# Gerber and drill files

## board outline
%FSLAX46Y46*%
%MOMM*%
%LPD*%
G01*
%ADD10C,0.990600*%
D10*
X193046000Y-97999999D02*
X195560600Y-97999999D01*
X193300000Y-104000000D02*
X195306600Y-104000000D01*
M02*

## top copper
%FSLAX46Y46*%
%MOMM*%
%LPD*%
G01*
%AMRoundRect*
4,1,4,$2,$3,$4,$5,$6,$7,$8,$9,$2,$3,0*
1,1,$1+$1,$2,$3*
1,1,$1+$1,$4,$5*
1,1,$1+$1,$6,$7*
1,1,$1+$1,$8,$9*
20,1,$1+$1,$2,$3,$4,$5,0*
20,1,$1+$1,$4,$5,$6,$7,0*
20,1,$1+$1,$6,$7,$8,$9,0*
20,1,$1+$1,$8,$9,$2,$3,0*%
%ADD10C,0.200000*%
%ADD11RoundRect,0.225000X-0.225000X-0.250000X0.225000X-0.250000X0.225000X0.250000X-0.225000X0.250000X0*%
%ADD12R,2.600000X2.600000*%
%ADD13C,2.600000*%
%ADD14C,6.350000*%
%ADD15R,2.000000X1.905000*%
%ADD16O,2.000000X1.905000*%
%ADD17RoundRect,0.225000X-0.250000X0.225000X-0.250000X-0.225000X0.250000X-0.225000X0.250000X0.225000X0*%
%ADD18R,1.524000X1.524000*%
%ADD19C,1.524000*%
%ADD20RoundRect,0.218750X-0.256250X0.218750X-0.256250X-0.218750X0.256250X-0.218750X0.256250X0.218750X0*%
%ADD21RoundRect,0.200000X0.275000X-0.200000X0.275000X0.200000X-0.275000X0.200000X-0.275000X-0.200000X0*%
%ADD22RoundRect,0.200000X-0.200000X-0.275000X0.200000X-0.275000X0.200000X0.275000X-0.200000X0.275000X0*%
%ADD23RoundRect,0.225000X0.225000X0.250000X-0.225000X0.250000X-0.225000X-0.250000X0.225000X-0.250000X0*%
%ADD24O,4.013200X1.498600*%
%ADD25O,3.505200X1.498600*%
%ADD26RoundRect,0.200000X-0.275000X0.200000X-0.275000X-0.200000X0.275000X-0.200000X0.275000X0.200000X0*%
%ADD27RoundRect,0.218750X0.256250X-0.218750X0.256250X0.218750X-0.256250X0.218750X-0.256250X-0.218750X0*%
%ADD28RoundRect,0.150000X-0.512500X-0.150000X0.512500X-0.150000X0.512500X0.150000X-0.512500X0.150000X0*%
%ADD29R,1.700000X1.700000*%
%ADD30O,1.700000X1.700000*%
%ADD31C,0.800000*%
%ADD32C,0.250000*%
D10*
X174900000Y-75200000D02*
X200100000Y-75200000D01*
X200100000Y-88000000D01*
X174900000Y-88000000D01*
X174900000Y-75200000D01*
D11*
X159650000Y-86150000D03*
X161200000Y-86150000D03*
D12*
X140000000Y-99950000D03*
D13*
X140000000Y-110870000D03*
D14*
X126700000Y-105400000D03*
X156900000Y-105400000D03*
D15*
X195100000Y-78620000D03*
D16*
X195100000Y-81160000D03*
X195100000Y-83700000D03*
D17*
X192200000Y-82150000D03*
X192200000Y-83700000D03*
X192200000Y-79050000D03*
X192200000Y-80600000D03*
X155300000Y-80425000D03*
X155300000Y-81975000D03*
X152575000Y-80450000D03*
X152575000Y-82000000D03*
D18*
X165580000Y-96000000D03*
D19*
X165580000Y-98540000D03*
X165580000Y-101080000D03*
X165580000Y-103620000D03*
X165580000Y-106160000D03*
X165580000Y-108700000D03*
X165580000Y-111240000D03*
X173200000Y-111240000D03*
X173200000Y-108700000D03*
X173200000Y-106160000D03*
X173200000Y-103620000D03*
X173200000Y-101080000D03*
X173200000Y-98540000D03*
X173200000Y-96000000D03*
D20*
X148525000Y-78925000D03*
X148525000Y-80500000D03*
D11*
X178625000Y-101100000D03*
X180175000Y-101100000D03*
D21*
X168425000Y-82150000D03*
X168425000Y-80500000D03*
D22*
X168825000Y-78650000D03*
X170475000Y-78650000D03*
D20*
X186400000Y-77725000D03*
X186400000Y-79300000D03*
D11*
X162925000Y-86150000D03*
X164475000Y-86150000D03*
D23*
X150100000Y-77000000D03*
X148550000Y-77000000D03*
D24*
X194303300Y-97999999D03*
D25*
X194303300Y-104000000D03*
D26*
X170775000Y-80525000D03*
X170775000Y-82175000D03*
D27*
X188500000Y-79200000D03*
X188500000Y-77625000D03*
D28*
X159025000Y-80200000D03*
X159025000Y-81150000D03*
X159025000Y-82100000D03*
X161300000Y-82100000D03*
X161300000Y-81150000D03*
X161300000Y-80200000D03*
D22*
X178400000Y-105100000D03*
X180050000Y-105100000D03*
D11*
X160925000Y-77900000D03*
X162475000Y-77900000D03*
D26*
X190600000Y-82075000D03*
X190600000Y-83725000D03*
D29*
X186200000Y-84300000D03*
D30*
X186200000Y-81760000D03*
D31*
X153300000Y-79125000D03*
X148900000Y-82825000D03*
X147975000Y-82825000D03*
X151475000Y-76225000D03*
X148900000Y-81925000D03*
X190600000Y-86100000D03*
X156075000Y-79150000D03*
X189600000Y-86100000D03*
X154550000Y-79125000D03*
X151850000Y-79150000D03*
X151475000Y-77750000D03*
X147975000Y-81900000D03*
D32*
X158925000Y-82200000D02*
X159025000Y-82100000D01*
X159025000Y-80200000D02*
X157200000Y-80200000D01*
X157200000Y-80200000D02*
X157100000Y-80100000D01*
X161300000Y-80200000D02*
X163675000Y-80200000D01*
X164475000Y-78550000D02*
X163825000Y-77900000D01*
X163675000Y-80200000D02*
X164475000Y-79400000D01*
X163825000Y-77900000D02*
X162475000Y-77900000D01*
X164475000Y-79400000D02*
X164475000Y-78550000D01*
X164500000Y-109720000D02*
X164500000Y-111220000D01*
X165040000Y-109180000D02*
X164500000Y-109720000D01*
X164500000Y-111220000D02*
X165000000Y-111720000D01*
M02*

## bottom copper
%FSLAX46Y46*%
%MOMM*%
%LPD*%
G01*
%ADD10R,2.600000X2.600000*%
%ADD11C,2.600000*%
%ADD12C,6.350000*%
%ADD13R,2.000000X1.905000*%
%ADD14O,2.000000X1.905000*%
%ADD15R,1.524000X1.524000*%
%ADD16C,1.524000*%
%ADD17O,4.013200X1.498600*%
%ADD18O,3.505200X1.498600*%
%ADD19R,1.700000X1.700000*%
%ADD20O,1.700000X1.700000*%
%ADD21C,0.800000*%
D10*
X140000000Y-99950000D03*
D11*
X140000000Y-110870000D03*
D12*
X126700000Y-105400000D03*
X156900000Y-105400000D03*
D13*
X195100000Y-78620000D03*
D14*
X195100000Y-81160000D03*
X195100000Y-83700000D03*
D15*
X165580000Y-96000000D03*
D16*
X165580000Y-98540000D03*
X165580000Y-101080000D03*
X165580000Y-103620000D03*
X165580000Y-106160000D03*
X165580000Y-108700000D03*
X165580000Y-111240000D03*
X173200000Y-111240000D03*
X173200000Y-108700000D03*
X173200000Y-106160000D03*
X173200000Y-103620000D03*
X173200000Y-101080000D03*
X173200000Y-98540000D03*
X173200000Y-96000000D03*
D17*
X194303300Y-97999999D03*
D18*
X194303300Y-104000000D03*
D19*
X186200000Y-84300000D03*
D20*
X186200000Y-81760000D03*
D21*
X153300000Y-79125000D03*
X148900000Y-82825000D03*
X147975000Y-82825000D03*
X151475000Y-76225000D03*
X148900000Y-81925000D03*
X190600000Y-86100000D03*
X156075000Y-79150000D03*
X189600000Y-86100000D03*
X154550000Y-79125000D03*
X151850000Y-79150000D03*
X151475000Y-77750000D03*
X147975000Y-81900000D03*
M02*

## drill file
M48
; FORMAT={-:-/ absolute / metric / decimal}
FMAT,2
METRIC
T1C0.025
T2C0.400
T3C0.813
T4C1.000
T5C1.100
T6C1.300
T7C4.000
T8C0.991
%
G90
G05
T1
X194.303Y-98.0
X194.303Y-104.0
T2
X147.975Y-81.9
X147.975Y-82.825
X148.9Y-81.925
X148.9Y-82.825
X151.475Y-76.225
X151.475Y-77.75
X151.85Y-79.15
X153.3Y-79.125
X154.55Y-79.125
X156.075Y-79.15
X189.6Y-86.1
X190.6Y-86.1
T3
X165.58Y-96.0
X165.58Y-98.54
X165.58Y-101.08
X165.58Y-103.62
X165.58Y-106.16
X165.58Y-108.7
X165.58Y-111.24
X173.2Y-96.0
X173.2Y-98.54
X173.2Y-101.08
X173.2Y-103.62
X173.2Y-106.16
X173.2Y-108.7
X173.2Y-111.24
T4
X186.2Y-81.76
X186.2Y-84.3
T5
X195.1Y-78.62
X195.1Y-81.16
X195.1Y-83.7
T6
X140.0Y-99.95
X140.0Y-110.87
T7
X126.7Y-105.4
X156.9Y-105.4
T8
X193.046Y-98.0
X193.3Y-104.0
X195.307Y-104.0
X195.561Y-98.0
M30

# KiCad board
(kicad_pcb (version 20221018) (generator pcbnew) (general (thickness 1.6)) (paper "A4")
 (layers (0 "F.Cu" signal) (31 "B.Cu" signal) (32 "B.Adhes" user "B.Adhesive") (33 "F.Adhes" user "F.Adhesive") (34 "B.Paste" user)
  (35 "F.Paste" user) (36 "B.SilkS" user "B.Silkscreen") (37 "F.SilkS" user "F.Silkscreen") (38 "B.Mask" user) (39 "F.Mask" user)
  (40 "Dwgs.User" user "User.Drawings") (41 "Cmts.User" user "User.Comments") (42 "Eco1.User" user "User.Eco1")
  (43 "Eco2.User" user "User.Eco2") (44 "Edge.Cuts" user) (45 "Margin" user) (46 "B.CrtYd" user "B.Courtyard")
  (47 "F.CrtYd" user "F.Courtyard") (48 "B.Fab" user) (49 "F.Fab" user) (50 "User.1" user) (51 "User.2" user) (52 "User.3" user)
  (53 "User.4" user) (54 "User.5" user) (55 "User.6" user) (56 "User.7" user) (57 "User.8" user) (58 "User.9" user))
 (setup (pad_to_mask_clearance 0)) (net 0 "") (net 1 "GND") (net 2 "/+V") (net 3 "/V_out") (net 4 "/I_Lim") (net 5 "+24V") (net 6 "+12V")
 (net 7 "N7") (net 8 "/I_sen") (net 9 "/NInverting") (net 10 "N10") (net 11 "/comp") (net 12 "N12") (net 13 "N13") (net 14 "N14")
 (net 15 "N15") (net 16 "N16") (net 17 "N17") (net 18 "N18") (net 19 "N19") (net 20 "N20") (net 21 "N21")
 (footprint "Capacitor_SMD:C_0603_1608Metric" (layer "F.Cu") (at 160.425 86.15)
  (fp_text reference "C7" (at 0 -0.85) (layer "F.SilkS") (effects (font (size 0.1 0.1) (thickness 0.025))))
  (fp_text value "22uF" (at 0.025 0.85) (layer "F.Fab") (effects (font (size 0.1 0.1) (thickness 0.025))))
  (pad "1" smd roundrect (at -0.775 0) (size 0.9 0.95) (layers "F.Cu" "F.Paste" "F.Mask") (roundrect_rratio 0.25) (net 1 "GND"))
  (pad "2" smd roundrect (at 0.775 0) (size 0.9 0.95) (layers "F.Cu" "F.Paste" "F.Mask") (roundrect_rratio 0.25) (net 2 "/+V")))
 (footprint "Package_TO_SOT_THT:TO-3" (layer "F.Cu") (at 140 99.95)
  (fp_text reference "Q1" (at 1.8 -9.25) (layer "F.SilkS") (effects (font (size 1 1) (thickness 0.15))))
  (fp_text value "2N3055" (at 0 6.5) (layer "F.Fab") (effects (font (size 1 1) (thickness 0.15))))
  (pad "1" thru_hole rect (at 0 0) (size 2.6 2.6) (drill 1.3) (layers "*.Cu" "*.Mask") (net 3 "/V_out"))
  (pad "2" thru_hole circle (at 0 10.92) (size 2.6 2.6) (drill 1.3) (layers "*.Cu" "*.Mask") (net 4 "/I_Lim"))
  (pad "3" thru_hole circle (at -13.3 5.45) (size 6.35 6.35) (drill 4) (layers "*.Cu" "*.Mask") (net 2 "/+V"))
  (pad "3" thru_hole circle (at 16.9 5.45) (size 6.35 6.35) (drill 4) (layers "*.Cu" "*.Mask") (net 2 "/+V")))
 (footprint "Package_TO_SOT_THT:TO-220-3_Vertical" (layer "F.Cu") (at 195.1 78.62 -90)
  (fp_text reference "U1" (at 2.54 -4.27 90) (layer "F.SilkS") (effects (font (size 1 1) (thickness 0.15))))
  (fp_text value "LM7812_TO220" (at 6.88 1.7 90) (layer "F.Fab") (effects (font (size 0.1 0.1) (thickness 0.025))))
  (pad "1" thru_hole rect (at 0 0 270) (size 1.905 2) (drill 1.1) (layers "*.Cu" "*.Mask") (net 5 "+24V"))
  (pad "2" thru_hole oval (at 2.54 0 270) (size 1.905 2) (drill 1.1) (layers "*.Cu" "*.Mask") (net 1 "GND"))
  (pad "3" thru_hole oval (at 5.08 0 270) (size 1.905 2) (drill 1.1) (layers "*.Cu" "*.Mask") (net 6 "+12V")))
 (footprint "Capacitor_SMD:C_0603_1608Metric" (layer "F.Cu") (at 192.2 82.925 -90)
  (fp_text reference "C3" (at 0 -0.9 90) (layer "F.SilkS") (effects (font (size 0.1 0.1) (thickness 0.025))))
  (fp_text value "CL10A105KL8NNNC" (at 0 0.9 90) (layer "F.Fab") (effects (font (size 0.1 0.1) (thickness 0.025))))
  (pad "1" smd roundrect (at -0.775 0 270) (size 0.9 0.95) (layers "F.Cu" "F.Paste" "F.Mask") (roundrect_rratio 0.25) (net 1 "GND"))
  (pad "2" smd roundrect (at 0.775 0 270) (size 0.9 0.95) (layers "F.Cu" "F.Paste" "F.Mask") (roundrect_rratio 0.25) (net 6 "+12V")))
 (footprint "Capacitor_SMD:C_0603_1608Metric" (layer "F.Cu") (at 192.2 79.825 -90)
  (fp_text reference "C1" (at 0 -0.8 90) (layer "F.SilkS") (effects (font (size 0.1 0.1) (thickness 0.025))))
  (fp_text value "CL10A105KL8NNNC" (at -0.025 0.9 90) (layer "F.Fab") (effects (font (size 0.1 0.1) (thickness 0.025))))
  (pad "1" smd roundrect (at -0.775 0 270) (size 0.9 0.95) (layers "F.Cu" "F.Paste" "F.Mask") (roundrect_rratio 0.25) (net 5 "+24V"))
  (pad "2" smd roundrect (at 0.775 0 270) (size 0.9 0.95) (layers "F.Cu" "F.Paste" "F.Mask") (roundrect_rratio 0.25) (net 1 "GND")))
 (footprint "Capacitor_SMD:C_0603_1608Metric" (layer "F.Cu") (at 155.3 81.2 -90)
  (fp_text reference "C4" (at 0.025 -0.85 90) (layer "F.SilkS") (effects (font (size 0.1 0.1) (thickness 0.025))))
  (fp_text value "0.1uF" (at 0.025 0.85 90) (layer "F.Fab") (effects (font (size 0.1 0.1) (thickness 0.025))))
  (pad "1" smd roundrect (at -0.775 0 270) (size 0.9 0.95) (layers "F.Cu" "F.Paste" "F.Mask") (roundrect_rratio 0.25) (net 1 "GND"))
  (pad "2" smd roundrect (at 0.775 0 270) (size 0.9 0.95) (layers "F.Cu" "F.Paste" "F.Mask") (roundrect_rratio 0.25) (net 5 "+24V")))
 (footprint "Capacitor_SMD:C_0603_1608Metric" (layer "F.Cu") (at 152.575 81.225 -90)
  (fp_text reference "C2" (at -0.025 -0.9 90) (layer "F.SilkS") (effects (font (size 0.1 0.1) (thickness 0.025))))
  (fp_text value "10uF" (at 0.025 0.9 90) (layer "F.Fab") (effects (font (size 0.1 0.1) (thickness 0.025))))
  (pad "1" smd roundrect (at -0.775 0 270) (size 0.9 0.95) (layers "F.Cu" "F.Paste" "F.Mask") (roundrect_rratio 0.25) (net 1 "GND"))
  (pad "2" smd roundrect (at 0.775 0 270) (size 0.9 0.95) (layers "F.Cu" "F.Paste" "F.Mask") (roundrect_rratio 0.25) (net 5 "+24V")))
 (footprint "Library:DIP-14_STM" (layer "F.Cu") (at 165.58 96)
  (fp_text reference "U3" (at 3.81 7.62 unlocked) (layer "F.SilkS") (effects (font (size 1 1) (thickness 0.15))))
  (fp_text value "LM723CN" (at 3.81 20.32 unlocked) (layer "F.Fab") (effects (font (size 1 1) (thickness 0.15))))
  (pad "1" thru_hole rect (at 0 0) (size 1.524 1.524) (drill 0.8128) (layers "*.Cu" "*.Mask") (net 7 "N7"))
  (pad "2" thru_hole circle (at 0 2.54) (size 1.524 1.524) (drill 0.8128) (layers "*.Cu" "*.Mask") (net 4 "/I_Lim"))
  (pad "3" thru_hole circle (at 0 5.08) (size 1.524 1.524) (drill 0.8128) (layers "*.Cu" "*.Mask") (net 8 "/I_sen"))
  (pad "4" thru_hole circle (at 0 7.62) (size 1.524 1.524) (drill 0.8128) (layers "*.Cu" "*.Mask") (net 1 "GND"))
  (pad "5" thru_hole circle (at 0 10.16) (size 1.524 1.524) (drill 0.8128) (layers "*.Cu" "*.Mask") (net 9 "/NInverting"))
  (pad "6" thru_hole circle (at 0 12.7) (size 1.524 1.524) (drill 0.8128) (layers "*.Cu" "*.Mask") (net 9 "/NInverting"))
  (pad "7" thru_hole circle (at 0 15.24) (size 1.524 1.524) (drill 0.8128) (layers "*.Cu" "*.Mask") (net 1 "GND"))
  (pad "8" thru_hole circle (at 7.62 15.24) (size 1.524 1.524) (drill 0.8128) (layers "*.Cu" "*.Mask") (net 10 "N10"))
  (pad "9" thru_hole circle (at 7.62 12.7) (size 1.524 1.524) (drill 0.8128) (layers "*.Cu" "*.Mask") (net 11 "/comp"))
  (pad "10" thru_hole circle (at 7.62 10.16) (size 1.524 1.524) (drill 0.8128) (layers "*.Cu" "*.Mask") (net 2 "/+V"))
  (pad "11" thru_hole circle (at 7.62 7.62) (size 1.524 1.524) (drill 0.8128) (layers "*.Cu" "*.Mask") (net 2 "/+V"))
  (pad "12" thru_hole circle (at 7.62 5.08) (size 1.524 1.524) (drill 0.8128) (layers "*.Cu" "*.Mask") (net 3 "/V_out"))
  (pad "13" thru_hole circle (at 7.62 2.54) (size 1.524 1.524) (drill 0.8128) (layers "*.Cu" "*.Mask") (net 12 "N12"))
  (pad "14" thru_hole circle (at 7.62 0) (size 1.524 1.524) (drill 0.8128) (layers "*.Cu" "*.Mask") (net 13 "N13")))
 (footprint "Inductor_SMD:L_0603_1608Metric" (layer "F.Cu") (at 148.525 79.7125 -90)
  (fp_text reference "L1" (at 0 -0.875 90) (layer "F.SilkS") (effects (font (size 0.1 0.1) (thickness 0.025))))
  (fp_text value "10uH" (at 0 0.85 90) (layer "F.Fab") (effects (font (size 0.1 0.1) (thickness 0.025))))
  (pad "1" smd roundrect (at -0.7875 0 270) (size 0.875 0.95) (layers "F.Cu" "F.Paste" "F.Mask") (roundrect_rratio 0.25) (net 2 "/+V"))
  (pad "2" smd roundrect (at 0.7875 0 270) (size 0.875 0.95) (layers "F.Cu" "F.Paste" "F.Mask") (roundrect_rratio 0.25) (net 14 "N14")))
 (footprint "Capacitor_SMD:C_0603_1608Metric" (layer "F.Cu") (at 179.4 101.1)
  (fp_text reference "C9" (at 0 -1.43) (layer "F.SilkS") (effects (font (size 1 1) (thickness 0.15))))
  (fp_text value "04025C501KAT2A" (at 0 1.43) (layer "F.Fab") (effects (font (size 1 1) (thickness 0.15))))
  (pad "1" smd roundrect (at -0.775 0) (size 0.9 0.95) (layers "F.Cu" "F.Paste" "F.Mask") (roundrect_rratio 0.25) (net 11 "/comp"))
  (pad "2" smd roundrect (at 0.775 0) (size 0.9 0.95) (layers "F.Cu" "F.Paste" "F.Mask") (roundrect_rratio 0.25) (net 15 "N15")))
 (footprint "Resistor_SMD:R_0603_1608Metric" (layer "F.Cu") (at 168.425 81.325 90)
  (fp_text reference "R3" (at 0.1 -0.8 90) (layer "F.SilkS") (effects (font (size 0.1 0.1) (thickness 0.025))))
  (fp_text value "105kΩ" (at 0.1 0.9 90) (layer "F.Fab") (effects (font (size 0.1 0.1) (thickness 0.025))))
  (pad "1" smd roundrect (at -0.825 0 90) (size 0.8 0.95) (layers "F.Cu" "F.Paste" "F.Mask") (roundrect_rratio 0.25) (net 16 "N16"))
  (pad "2" smd roundrect (at 0.825 0 90) (size 0.8 0.95) (layers "F.Cu" "F.Paste" "F.Mask") (roundrect_rratio 0.25) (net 1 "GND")))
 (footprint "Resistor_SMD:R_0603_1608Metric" (layer "F.Cu") (at 169.65 78.65)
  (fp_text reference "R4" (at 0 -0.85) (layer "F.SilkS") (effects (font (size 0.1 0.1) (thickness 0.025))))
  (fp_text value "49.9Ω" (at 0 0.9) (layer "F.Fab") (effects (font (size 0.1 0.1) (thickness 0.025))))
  (pad "1" smd roundrect (at -0.825 0) (size 0.8 0.95) (layers "F.Cu" "F.Paste" "F.Mask") (roundrect_rratio 0.25) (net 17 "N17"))
  (pad "2" smd roundrect (at 0.825 0) (size 0.8 0.95) (layers "F.Cu" "F.Paste" "F.Mask") (roundrect_rratio 0.25) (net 2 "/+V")))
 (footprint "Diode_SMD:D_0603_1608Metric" (layer "F.Cu") (at 186.4 78.5125 -90)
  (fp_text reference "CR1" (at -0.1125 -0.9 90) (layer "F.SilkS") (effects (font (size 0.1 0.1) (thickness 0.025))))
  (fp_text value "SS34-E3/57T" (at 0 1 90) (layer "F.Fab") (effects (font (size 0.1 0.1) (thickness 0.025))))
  (pad "1" smd roundrect (at -0.7875 0 270) (size 0.875 0.95) (layers "F.Cu" "F.Paste" "F.Mask") (roundrect_rratio 0.25) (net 6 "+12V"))
  (pad "2" smd roundrect (at 0.7875 0 270) (size 0.875 0.95) (layers "F.Cu" "F.Paste" "F.Mask") (roundrect_rratio 0.25) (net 1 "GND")))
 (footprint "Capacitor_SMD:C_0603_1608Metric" (layer "F.Cu") (at 163.7 86.15)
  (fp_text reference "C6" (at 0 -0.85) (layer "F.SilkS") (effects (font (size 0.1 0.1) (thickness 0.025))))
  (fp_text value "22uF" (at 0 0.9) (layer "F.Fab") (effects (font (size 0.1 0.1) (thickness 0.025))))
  (pad "1" smd roundrect (at -0.775 0) (size 0.9 0.95) (layers "F.Cu" "F.Paste" "F.Mask") (roundrect_rratio 0.25) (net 1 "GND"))
  (pad "2" smd roundrect (at 0.775 0) (size 0.9 0.95) (layers "F.Cu" "F.Paste" "F.Mask") (roundrect_rratio 0.25) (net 2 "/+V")))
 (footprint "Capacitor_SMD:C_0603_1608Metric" (layer "F.Cu") (at 149.325 77 180)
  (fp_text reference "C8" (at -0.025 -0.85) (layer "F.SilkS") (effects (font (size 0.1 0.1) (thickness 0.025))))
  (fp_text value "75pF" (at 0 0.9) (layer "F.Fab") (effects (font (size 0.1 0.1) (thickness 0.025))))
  (pad "1" smd roundrect (at -0.775 0 180) (size 0.9 0.95) (layers "F.Cu" "F.Paste" "F.Mask") (roundrect_rratio 0.25) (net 1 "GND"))
  (pad "2" smd roundrect (at 0.775 0 180) (size 0.9 0.95) (layers "F.Cu" "F.Paste" "F.Mask") (roundrect_rratio 0.25) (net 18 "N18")))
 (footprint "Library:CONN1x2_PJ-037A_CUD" (layer "F.Cu") (at 194.3033 97.999999)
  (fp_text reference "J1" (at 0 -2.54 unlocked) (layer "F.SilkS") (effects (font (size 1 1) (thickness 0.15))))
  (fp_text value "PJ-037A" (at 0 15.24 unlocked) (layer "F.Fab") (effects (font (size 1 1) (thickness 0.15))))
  (fp_line (start -1.2573 0) (end 1.2573 0) (stroke (width 0.9906) (type solid)) (layer "Edge.Cuts"))
  (fp_line (start -1.0033 6.000001) (end 1.0033 6.000001) (stroke (width 0.9906) (type solid)) (layer "Edge.Cuts"))
  (pad "" np_thru_hole circle (at -1.2573 0) (size 0.9906 0.9906) (drill 0.9906) (layers "*.Cu" "*.Mask"))
  (pad "" np_thru_hole circle (at -1.0033 6.000001) (size 0.9906 0.9906) (drill 0.9906) (layers "*.Cu" "*.Mask"))
  (pad "" np_thru_hole circle (at 1.0033 6.000001) (size 0.9906 0.9906) (drill 0.9906) (layers "*.Cu" "*.Mask"))
  (pad "" np_thru_hole circle (at 1.2573 0) (size 0.9906 0.9906) (drill 0.9906) (layers "*.Cu" "*.Mask"))
  (pad "1" thru_hole oval (at 0 0) (size 4.0132 1.4986) (drill 0.0254) (layers "*.Cu" "*.Mask") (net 1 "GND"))
  (pad "2" thru_hole oval (at 0 6.000001) (size 3.5052 1.4986) (drill 0.0254) (layers "*.Cu" "*.Mask") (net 5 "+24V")))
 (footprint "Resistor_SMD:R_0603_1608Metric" (layer "F.Cu") (at 170.775 81.35 -90)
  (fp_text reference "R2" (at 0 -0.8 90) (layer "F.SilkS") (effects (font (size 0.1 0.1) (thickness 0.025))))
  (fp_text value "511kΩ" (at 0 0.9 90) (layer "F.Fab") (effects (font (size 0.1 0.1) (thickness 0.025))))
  (pad "1" smd roundrect (at -0.825 0 270) (size 0.8 0.95) (layers "F.Cu" "F.Paste" "F.Mask") (roundrect_rratio 0.25) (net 5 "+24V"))
  (pad "2" smd roundrect (at 0.825 0 270) (size 0.8 0.95) (layers "F.Cu" "F.Paste" "F.Mask") (roundrect_rratio 0.25) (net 16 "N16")))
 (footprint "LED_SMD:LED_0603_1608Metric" (layer "F.Cu") (at 188.5 78.4125 90)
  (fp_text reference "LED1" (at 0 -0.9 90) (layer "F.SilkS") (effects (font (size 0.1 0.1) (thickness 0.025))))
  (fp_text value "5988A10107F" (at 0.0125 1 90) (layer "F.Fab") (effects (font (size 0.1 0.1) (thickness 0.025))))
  (pad "1" smd roundrect (at -0.7875 0 90) (size 0.875 0.95) (layers "F.Cu" "F.Paste" "F.Mask") (roundrect_rratio 0.25) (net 1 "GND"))
  (pad "2" smd roundrect (at 0.7875 0 90) (size 0.875 0.95) (layers "F.Cu" "F.Paste" "F.Mask") (roundrect_rratio 0.25) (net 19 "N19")))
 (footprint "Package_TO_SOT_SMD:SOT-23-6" (layer "F.Cu") (at 160.1625 81.15)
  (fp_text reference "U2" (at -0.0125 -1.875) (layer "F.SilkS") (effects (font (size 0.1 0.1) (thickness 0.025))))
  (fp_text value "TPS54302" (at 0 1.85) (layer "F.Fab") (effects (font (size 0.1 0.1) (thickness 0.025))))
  (pad "1" smd roundrect (at -1.1375 -0.95) (size 1.325 0.6) (layers "F.Cu" "F.Paste" "F.Mask") (roundrect_rratio 0.25) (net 1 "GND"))
  (pad "2" smd roundrect (at -1.1375 0) (size 1.325 0.6) (layers "F.Cu" "F.Paste" "F.Mask") (roundrect_rratio 0.25) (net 14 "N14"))
  (pad "3" smd roundrect (at -1.1375 0.95) (size 1.325 0.6) (layers "F.Cu" "F.Paste" "F.Mask") (roundrect_rratio 0.25) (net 5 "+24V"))
  (pad "4" smd roundrect (at 1.1375 0.95) (size 1.325 0.6) (layers "F.Cu" "F.Paste" "F.Mask") (roundrect_rratio 0.25) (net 1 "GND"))
  (pad "5" smd roundrect (at 1.1375 0) (size 1.325 0.6) (layers "F.Cu" "F.Paste" "F.Mask") (roundrect_rratio 0.25) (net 16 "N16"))
  (pad "6" smd roundrect (at 1.1375 -0.95) (size 1.325 0.6) (layers "F.Cu" "F.Paste" "F.Mask") (roundrect_rratio 0.25) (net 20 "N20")))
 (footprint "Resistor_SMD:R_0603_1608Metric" (layer "F.Cu") (at 179.225 105.1)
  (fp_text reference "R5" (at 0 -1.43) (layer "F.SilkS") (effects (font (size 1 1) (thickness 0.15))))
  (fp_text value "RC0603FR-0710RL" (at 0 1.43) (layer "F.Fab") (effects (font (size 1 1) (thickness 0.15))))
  (pad "1" smd roundrect (at -0.825 0) (size 0.8 0.95) (layers "F.Cu" "F.Paste" "F.Mask") (roundrect_rratio 0.25) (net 4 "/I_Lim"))
  (pad "2" smd roundrect (at 0.825 0) (size 0.8 0.95) (layers "F.Cu" "F.Paste" "F.Mask") (roundrect_rratio 0.25) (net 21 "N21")))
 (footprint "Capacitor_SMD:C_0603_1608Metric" (layer "F.Cu") (at 161.7 77.9)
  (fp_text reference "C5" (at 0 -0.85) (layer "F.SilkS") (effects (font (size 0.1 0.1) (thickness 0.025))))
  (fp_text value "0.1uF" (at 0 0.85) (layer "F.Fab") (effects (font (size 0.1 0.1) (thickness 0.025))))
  (pad "1" smd roundrect (at -0.775 0) (size 0.9 0.95) (layers "F.Cu" "F.Paste" "F.Mask") (roundrect_rratio 0.25) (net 14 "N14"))
  (pad "2" smd roundrect (at 0.775 0) (size 0.9 0.95) (layers "F.Cu" "F.Paste" "F.Mask") (roundrect_rratio 0.25) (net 20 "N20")))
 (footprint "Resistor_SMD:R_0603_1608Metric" (layer "F.Cu") (at 190.6 82.9 -90)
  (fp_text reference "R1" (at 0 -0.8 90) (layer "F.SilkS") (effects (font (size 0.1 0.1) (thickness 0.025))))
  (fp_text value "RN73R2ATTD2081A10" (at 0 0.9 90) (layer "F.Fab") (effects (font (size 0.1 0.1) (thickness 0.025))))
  (pad "1" smd roundrect (at -0.825 0 270) (size 0.8 0.95) (layers "F.Cu" "F.Paste" "F.Mask") (roundrect_rratio 0.25) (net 19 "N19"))
  (pad "2" smd roundrect (at 0.825 0 270) (size 0.8 0.95) (layers "F.Cu" "F.Paste" "F.Mask") (roundrect_rratio 0.25) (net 6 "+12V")))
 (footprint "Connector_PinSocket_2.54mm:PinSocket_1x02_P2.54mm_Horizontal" (layer "B.Cu") (at 186.2 84.3)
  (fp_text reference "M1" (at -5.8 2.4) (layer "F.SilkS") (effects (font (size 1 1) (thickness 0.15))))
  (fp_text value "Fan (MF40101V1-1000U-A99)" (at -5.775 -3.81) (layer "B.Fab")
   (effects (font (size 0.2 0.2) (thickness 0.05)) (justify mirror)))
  (pad "1" thru_hole rect (at 0 0) (size 1.7 1.7) (drill 1) (layers "*.Cu" "*.Mask") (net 6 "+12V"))
  (pad "2" thru_hole oval (at 0 -2.54) (size 1.7 1.7) (drill 1) (layers "*.Cu" "*.Mask") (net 1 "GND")))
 (gr_rect (start 174.9 75.2) (end 200.1 88) (stroke (width 0.2) (type default)) (fill none) (layer "F.Cu"))
 (via (at 153.3 79.125) (size 0.8) (drill 0.4) (layers "F.Cu" "B.Cu") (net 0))
 (via (at 148.9 82.825) (size 0.8) (drill 0.4) (layers "F.Cu" "B.Cu") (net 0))
 (via (at 147.975 82.825) (size 0.8) (drill 0.4) (layers "F.Cu" "B.Cu") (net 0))
 (via (at 151.475 76.225) (size 0.8) (drill 0.4) (layers "F.Cu" "B.Cu") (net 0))
 (via (at 148.9 81.925) (size 0.8) (drill 0.4) (layers "F.Cu" "B.Cu") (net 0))
 (via (at 190.6 86.1) (size 0.8) (drill 0.4) (layers "F.Cu" "B.Cu") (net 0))
 (via (at 156.075 79.15) (size 0.8) (drill 0.4) (layers "F.Cu" "B.Cu") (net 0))
 (via (at 189.6 86.1) (size 0.8) (drill 0.4) (layers "F.Cu" "B.Cu") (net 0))
 (via (at 154.55 79.125) (size 0.8) (drill 0.4) (layers "F.Cu" "B.Cu") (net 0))
 (via (at 151.85 79.15) (size 0.8) (drill 0.4) (layers "F.Cu" "B.Cu") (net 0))
 (via (at 151.475 77.75) (size 0.8) (drill 0.4) (layers "F.Cu" "B.Cu") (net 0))
 (via (at 147.975 81.9) (size 0.8) (drill 0.4) (layers "F.Cu" "B.Cu") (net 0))
 (segment (start 158.925 82.2) (end 159.025 82.1) (width 0.25) (layer "F.Cu") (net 5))
 (segment (start 159.025 80.2) (end 157.2 80.2) (width 0.25) (layer "F.Cu") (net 1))
 (segment (start 157.2 80.2) (end 157.1 80.1) (width 0.25) (layer "F.Cu") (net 1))
 (segment (start 161.3 80.2) (end 163.675 80.2) (width 0.25) (layer "F.Cu") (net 20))
 (segment (start 164.475 78.55) (end 163.825 77.9) (width 0.25) (layer "F.Cu") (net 20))
 (segment (start 163.675 80.2) (end 164.475 79.4) (width 0.25) (layer "F.Cu") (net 20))
 (segment (start 163.825 77.9) (end 162.475 77.9) (width 0.25) (layer "F.Cu") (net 20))
 (segment (start 164.475 79.4) (end 164.475 78.55) (width 0.25) (layer "F.Cu") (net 20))
 (segment (start 164.5 109.72) (end 164.5 111.22) (width 0.25) (layer "F.Cu") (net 9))
 (segment (start 165.04 109.18) (end 164.5 109.72) (width 0.25) (layer "F.Cu") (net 9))
 (segment (start 164.5 111.22) (end 165 111.72) (width 0.25) (layer "F.Cu") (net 9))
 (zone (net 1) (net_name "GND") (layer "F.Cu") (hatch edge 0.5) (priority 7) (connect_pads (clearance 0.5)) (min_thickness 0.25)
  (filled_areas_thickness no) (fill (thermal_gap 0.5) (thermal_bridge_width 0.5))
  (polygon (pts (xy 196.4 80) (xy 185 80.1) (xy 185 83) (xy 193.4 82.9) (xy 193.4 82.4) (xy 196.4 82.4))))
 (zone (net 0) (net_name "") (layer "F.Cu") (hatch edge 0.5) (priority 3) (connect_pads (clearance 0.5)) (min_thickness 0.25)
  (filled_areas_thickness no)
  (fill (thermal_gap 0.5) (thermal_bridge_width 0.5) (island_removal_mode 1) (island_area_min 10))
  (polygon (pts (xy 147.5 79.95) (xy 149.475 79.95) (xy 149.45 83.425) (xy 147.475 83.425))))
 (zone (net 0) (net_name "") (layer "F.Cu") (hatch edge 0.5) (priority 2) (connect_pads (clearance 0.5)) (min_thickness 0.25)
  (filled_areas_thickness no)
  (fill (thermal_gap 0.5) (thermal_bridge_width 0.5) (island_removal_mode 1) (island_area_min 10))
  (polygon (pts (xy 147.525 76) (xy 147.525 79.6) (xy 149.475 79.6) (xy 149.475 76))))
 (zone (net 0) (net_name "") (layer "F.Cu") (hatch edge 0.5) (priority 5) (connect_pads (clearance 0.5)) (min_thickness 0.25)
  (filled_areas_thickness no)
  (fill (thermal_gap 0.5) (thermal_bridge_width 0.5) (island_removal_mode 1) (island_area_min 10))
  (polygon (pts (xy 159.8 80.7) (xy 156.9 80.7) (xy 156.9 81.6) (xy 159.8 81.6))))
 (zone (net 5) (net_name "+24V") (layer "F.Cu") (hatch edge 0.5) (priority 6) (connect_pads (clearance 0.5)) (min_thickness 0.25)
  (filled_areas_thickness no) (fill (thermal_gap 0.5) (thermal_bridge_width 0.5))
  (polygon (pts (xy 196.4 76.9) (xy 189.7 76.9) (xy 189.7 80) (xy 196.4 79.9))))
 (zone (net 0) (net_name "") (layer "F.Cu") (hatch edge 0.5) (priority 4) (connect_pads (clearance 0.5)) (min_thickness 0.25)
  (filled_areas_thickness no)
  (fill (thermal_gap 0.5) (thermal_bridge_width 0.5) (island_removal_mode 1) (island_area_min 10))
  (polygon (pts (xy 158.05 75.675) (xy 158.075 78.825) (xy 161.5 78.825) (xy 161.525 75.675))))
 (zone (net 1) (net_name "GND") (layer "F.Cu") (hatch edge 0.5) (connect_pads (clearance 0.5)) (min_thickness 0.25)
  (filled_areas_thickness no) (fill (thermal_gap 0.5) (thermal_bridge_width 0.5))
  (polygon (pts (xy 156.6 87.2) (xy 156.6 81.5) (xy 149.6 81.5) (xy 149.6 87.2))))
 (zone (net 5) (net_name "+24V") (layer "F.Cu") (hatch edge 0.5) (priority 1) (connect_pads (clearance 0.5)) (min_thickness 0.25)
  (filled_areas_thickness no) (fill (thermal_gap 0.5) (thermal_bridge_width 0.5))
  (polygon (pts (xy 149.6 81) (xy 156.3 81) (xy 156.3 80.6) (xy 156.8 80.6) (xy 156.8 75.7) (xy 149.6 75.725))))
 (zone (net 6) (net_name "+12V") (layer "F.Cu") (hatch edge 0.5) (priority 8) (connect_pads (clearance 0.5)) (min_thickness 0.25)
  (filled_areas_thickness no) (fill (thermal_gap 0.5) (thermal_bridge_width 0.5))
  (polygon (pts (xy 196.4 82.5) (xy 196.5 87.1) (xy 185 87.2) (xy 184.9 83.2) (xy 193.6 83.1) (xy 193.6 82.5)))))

